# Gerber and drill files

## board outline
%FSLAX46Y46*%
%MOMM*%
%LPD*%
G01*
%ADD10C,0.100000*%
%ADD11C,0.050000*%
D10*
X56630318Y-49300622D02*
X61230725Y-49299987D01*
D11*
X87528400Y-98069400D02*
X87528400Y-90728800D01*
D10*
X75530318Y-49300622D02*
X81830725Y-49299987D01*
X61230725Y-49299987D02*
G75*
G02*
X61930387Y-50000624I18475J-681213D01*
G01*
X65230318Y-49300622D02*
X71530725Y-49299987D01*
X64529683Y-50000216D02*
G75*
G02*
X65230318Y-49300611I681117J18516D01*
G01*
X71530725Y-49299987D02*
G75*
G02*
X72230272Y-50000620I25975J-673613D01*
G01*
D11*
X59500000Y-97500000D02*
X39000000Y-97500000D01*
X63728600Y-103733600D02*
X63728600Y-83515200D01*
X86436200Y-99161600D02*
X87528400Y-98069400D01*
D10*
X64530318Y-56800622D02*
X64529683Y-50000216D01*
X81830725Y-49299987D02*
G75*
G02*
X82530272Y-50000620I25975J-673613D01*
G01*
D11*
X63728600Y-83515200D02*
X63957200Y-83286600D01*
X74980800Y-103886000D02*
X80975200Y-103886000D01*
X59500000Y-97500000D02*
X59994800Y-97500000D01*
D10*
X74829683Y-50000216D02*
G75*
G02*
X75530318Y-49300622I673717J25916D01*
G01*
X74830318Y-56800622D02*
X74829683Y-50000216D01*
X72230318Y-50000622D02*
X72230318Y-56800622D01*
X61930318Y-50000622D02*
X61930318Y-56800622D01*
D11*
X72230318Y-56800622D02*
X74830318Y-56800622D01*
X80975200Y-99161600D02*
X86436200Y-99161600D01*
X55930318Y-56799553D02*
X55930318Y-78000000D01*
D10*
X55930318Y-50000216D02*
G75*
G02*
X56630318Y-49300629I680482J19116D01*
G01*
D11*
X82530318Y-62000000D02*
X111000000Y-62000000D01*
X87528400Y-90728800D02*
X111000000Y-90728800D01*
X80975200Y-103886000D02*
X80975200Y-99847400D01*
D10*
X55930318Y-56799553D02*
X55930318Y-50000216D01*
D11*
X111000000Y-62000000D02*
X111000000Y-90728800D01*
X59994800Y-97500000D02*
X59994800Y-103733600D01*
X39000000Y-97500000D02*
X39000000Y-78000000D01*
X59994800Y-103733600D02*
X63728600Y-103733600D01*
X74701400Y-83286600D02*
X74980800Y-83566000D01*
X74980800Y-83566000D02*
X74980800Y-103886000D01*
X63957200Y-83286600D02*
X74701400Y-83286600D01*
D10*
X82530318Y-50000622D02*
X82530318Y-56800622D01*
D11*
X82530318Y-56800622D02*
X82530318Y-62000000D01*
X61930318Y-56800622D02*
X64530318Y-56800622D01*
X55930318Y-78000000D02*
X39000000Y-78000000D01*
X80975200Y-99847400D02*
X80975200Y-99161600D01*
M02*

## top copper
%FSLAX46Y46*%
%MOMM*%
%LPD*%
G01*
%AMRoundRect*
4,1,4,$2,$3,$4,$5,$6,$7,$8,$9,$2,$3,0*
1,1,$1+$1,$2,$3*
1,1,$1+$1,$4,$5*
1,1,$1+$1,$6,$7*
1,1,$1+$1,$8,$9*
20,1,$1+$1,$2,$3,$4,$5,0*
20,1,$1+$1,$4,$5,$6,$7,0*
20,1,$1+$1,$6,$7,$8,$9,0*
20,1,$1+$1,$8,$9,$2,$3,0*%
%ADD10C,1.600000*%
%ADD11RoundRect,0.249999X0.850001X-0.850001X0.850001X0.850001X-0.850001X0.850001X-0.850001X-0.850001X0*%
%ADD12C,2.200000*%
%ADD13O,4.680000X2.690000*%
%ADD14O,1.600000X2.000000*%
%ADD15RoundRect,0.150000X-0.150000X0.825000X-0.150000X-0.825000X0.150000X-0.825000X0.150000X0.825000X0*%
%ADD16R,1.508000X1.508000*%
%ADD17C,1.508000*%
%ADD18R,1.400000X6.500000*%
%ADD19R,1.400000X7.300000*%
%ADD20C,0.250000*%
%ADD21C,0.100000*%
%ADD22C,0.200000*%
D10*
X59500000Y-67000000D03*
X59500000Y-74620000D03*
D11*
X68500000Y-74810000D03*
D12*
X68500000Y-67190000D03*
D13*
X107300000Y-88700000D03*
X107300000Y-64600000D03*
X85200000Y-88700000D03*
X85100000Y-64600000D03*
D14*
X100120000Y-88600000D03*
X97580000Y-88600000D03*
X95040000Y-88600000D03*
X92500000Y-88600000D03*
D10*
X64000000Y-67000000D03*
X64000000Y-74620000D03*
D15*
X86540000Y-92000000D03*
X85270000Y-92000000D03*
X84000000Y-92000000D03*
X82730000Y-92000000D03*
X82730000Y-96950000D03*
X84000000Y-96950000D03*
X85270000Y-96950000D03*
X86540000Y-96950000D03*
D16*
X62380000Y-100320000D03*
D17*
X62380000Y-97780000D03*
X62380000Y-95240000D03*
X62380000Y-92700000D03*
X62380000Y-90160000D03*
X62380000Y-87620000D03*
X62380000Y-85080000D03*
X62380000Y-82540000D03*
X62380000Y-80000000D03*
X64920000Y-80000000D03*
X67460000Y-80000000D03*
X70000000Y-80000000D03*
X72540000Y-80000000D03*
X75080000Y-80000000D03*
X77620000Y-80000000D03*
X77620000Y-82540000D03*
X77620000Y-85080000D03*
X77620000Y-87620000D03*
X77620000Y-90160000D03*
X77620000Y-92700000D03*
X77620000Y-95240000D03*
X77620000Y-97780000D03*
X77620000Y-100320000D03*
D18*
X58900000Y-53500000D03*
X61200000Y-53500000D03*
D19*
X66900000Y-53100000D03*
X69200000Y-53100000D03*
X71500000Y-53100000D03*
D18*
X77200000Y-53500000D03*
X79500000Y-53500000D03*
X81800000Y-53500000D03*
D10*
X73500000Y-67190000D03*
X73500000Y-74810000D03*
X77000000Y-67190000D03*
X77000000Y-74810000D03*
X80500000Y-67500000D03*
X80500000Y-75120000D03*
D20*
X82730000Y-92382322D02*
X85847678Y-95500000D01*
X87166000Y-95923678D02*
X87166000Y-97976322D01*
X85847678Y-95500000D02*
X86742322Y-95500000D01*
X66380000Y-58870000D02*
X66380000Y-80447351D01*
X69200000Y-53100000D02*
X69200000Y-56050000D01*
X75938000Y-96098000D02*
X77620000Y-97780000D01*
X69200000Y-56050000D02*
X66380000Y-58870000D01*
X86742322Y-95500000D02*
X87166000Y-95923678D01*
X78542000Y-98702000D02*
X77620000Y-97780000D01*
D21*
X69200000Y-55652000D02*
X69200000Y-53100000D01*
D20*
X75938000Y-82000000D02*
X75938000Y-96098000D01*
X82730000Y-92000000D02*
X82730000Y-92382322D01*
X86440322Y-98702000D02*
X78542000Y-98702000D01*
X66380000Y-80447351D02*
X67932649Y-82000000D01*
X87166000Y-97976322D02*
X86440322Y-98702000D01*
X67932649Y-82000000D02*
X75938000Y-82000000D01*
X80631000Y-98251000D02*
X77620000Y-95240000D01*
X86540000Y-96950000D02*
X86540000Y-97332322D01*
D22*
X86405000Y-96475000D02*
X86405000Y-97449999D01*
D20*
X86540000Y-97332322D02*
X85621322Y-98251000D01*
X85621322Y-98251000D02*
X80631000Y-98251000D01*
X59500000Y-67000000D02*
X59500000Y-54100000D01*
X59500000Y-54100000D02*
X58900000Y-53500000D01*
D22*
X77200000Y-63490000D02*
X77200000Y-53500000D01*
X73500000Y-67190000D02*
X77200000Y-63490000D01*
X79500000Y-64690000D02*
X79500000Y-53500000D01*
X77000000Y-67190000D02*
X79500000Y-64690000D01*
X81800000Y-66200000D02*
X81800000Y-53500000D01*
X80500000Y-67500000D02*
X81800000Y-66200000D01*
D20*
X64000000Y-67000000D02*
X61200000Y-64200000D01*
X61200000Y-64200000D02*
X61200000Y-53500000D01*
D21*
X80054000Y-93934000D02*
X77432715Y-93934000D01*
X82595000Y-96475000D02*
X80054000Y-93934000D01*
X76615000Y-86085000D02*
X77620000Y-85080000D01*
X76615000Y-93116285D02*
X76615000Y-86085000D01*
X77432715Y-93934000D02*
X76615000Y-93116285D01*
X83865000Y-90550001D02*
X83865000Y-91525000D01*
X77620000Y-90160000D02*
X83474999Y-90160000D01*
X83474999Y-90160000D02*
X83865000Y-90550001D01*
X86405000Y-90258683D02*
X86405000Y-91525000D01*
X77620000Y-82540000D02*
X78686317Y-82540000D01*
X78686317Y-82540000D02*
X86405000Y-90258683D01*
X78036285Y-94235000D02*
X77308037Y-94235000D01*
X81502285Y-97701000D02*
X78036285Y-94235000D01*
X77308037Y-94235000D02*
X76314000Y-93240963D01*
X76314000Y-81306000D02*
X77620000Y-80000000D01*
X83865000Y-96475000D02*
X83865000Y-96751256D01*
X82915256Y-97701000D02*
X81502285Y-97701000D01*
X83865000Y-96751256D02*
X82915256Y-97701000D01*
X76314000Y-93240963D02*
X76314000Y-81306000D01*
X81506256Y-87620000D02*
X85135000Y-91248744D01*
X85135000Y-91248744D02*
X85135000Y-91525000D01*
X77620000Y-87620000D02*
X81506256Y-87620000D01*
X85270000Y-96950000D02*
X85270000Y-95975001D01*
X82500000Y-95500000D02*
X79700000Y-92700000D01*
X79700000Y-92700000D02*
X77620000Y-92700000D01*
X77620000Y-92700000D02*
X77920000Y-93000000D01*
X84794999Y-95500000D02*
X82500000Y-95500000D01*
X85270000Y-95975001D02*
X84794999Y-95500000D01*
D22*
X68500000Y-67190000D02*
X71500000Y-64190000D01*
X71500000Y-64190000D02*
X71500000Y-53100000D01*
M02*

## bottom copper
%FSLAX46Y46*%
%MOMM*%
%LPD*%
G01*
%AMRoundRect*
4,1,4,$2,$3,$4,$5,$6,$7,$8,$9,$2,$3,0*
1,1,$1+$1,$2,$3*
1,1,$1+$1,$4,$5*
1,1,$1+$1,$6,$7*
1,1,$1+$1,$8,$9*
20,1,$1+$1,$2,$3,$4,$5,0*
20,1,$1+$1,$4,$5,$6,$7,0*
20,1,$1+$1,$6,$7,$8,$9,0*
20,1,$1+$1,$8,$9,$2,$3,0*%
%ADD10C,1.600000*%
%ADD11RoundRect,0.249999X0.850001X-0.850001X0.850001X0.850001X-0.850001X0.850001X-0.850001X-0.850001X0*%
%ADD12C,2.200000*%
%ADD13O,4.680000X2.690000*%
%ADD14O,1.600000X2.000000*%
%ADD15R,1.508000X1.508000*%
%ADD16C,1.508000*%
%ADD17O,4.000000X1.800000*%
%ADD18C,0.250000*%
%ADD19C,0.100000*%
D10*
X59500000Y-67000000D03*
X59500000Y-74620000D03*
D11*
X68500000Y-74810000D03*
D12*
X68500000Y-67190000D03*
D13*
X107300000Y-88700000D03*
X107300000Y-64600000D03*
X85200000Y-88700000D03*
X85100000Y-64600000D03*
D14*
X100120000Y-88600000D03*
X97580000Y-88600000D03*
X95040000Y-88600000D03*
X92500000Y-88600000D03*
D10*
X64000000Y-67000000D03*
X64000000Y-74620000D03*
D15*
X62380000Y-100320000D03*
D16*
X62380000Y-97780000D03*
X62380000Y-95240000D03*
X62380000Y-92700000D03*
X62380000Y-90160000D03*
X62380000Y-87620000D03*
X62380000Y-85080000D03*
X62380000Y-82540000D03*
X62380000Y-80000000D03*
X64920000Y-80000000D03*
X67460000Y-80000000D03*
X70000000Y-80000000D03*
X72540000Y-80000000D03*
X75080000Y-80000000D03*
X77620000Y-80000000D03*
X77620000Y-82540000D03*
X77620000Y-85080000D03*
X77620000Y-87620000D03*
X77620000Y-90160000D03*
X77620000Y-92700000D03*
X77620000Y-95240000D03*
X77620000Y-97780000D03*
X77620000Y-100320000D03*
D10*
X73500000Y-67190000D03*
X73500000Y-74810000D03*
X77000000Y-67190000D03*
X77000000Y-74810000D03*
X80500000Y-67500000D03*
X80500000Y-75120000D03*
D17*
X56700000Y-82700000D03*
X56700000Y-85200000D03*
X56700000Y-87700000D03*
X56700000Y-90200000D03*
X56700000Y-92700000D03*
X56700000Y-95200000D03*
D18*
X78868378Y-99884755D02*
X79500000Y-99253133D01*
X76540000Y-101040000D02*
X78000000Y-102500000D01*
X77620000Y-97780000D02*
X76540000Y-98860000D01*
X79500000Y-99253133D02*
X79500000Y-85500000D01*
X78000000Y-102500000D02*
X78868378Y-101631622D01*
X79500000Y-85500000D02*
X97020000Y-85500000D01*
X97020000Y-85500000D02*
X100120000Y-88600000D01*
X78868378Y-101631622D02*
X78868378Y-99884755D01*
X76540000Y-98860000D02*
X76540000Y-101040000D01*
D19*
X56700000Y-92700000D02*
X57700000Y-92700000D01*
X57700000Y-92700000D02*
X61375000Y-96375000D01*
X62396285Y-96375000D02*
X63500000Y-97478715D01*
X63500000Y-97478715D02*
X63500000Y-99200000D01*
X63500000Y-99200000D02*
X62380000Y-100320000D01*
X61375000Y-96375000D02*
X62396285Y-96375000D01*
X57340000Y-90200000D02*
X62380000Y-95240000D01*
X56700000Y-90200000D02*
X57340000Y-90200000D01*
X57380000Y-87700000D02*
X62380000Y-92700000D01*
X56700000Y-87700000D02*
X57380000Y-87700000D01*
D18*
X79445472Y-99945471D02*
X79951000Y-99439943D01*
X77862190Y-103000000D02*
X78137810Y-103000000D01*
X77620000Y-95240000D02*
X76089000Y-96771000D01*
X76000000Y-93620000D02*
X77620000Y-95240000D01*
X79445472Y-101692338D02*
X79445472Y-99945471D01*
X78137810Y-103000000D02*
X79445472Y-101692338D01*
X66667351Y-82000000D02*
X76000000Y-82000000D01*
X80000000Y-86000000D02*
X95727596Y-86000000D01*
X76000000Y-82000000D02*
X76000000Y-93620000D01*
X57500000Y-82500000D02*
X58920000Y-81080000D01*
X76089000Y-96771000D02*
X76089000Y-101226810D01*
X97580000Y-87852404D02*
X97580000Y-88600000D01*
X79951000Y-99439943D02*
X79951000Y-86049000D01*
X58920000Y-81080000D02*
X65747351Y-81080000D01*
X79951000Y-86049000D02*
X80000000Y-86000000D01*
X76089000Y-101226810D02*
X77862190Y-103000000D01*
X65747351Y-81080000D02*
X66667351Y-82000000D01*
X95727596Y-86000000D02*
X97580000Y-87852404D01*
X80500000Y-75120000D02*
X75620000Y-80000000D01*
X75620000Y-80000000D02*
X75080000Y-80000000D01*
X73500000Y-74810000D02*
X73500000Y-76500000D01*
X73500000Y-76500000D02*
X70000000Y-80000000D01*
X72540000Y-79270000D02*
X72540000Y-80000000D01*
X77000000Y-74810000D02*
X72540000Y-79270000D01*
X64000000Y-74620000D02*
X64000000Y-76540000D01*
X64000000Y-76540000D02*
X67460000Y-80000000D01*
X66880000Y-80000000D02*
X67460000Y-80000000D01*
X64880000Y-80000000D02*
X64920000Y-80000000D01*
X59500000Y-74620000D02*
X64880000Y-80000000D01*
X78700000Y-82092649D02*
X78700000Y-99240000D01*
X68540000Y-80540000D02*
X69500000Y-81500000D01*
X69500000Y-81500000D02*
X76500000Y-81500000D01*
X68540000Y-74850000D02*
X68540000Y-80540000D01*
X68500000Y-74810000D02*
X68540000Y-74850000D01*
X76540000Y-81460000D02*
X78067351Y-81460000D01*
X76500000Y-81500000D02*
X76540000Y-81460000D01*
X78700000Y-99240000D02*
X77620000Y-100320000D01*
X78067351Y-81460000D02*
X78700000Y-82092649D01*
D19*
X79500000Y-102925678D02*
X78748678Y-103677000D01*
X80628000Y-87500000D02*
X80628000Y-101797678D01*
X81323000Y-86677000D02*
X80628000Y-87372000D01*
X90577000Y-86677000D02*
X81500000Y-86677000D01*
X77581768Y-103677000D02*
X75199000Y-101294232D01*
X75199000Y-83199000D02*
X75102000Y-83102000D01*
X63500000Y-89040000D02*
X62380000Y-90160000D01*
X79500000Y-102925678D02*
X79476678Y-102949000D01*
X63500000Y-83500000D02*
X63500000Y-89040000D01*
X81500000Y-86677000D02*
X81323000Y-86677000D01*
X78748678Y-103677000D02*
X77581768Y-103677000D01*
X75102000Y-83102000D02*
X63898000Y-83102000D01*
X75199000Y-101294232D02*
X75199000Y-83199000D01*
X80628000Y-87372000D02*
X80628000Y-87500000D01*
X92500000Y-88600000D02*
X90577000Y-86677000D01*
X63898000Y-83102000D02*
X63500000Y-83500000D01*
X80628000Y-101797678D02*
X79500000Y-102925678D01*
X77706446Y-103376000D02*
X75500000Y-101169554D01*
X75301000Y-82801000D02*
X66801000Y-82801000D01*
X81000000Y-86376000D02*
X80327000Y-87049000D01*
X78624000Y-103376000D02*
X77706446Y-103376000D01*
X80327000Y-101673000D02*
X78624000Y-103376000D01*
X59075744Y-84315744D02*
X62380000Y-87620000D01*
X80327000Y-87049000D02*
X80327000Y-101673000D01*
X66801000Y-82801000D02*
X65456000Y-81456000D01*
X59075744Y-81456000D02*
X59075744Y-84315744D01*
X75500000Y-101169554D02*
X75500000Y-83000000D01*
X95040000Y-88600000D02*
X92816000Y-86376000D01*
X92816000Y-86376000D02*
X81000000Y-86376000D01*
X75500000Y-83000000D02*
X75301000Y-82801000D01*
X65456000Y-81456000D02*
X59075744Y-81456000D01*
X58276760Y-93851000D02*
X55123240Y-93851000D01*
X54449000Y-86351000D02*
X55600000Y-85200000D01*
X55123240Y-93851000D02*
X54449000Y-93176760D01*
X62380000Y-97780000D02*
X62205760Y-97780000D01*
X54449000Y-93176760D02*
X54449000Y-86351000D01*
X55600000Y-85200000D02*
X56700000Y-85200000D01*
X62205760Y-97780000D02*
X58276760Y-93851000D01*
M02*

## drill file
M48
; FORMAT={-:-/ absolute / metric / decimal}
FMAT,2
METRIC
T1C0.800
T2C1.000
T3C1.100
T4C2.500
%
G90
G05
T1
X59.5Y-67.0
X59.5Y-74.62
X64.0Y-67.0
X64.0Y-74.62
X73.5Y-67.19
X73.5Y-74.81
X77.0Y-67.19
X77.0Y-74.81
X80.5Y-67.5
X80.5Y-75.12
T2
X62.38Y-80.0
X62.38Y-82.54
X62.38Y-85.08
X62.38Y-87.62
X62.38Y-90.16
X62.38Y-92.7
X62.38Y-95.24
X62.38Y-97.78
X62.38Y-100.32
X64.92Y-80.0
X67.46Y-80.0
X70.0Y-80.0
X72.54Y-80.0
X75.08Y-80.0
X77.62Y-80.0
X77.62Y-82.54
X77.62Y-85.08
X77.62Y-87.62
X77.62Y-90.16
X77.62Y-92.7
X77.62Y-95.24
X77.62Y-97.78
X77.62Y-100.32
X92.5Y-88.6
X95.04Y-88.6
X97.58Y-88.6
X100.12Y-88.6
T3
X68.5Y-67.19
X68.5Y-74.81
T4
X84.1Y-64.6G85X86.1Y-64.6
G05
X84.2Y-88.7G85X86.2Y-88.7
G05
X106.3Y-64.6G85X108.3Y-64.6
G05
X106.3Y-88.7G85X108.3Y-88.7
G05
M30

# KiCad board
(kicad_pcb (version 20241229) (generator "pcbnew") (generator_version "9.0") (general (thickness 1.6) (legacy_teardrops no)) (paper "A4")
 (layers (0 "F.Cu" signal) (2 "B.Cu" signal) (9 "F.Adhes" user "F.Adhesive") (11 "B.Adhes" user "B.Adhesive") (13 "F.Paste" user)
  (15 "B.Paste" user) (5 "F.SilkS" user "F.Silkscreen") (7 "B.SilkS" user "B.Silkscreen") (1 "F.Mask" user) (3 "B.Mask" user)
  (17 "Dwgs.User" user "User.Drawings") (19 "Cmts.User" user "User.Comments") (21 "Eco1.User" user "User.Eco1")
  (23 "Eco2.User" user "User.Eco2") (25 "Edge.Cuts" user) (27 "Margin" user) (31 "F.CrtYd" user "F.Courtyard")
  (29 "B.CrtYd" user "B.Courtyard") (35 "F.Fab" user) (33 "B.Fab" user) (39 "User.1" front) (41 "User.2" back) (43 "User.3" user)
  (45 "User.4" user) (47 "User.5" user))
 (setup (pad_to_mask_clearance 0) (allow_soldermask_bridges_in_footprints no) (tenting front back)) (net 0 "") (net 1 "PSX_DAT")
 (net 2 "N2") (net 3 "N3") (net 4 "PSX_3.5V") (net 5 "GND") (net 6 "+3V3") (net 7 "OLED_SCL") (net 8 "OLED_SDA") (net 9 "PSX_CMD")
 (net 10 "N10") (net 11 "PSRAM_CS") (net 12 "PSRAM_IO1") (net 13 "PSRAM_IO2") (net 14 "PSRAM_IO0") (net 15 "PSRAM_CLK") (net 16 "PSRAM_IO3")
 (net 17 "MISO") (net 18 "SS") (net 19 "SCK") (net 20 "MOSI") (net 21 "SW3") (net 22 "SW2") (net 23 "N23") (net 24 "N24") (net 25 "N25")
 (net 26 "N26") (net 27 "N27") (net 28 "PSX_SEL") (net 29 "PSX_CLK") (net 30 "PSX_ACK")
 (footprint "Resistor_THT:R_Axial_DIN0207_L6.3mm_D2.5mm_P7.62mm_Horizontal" (layer "F.Cu") (at 59.5 67 -90)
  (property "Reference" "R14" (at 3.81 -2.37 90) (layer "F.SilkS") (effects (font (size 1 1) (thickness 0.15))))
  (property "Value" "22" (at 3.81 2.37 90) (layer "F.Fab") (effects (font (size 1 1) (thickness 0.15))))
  (pad "1" thru_hole circle (at 0 0 270) (size 1.6 1.6) (drill 0.8) (layers "*.Cu" "*.Mask") (remove_unused_layers no) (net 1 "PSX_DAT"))
  (pad "2" thru_hole circle (at 7.62 0 270) (size 1.6 1.6) (drill 0.8) (layers "*.Cu" "*.Mask") (remove_unused_layers no) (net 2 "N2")))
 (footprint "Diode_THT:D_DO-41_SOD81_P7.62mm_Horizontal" (layer "F.Cu") (at 68.5 74.81 90)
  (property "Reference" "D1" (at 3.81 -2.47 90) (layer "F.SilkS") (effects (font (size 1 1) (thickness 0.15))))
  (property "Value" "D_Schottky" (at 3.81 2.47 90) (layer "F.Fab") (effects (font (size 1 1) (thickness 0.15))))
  (pad "1" thru_hole roundrect (at 0 0 90) (size 2.2 2.2) (drill 1.1) (layers "*.Cu" "*.Mask") (remove_unused_layers no)
   (roundrect_rratio 0.113636) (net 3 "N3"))
  (pad "2" thru_hole circle (at 7.62 0 90) (size 2.2 2.2) (drill 1.1) (layers "*.Cu" "*.Mask") (remove_unused_layers no) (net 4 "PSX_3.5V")))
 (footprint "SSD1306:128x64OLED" (layer "F.Cu") (at 96.5 78 180)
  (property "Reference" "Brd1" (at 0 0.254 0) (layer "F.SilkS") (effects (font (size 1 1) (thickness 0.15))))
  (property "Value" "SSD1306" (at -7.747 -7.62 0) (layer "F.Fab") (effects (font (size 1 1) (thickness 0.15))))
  (pad "" thru_hole oval (at -10.8 -10.7) (size 4.68 2.69) (drill oval 4.5 2.5) (layers "*.Cu" "*.Mask") (remove_unused_layers no))
  (pad "" thru_hole oval (at -10.8 13.4) (size 4.68 2.69) (drill oval 4.5 2.5) (layers "*.Cu" "*.Mask") (remove_unused_layers no))
  (pad "" thru_hole oval (at 11.3 -10.7) (size 4.68 2.69) (drill oval 4.5 2.5) (layers "*.Cu" "*.Mask") (remove_unused_layers no))
  (pad "" thru_hole oval (at 11.4 13.4) (size 4.68 2.69) (drill oval 4.5 2.5) (layers "*.Cu" "*.Mask") (remove_unused_layers no))
  (pad "1" thru_hole oval (at -3.62 -10.6 270) (size 2 1.6) (drill 1) (layers "*.Cu" "*.Mask") (remove_unused_layers no) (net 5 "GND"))
  (pad "2" thru_hole oval (at -1.08 -10.6 270) (size 2 1.6) (drill 1) (layers "*.Cu" "*.Mask") (remove_unused_layers no) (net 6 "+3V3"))
  (pad "3" thru_hole oval (at 1.46 -10.6 270) (size 2 1.6) (drill 1) (layers "*.Cu" "*.Mask") (remove_unused_layers no) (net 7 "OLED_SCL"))
  (pad "4" thru_hole oval (at 4 -10.6 270) (size 2 1.6) (drill 1) (layers "*.Cu" "*.Mask") (remove_unused_layers no) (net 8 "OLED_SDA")))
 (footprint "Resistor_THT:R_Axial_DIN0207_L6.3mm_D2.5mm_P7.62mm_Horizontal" (layer "F.Cu") (at 64 67 -90)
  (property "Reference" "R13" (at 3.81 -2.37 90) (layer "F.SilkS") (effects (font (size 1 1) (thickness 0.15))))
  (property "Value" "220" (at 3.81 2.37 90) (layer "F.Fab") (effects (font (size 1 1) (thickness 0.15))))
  (pad "1" thru_hole circle (at 0 0 270) (size 1.6 1.6) (drill 0.8) (layers "*.Cu" "*.Mask") (remove_unused_layers no) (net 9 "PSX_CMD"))
  (pad "2" thru_hole circle (at 7.62 0 270) (size 1.6 1.6) (drill 0.8) (layers "*.Cu" "*.Mask") (remove_unused_layers no) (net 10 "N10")))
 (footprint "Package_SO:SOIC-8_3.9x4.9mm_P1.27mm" (layer "F.Cu") (at 84.635 94.475 -90)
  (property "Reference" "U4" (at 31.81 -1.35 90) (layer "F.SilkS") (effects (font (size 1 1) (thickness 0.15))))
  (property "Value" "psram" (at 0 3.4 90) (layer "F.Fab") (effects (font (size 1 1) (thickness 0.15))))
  (pad "1" smd roundrect (at -2.475 -1.905 270) (size 1.95 0.6) (layers "F.Cu" "F.Mask" "F.Paste") (roundrect_rratio 0.25)
   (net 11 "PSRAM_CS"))
  (pad "2" smd roundrect (at -2.475 -0.635 270) (size 1.95 0.6) (layers "F.Cu" "F.Mask" "F.Paste") (roundrect_rratio 0.25)
   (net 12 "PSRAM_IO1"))
  (pad "3" smd roundrect (at -2.475 0.635 270) (size 1.95 0.6) (layers "F.Cu" "F.Mask" "F.Paste") (roundrect_rratio 0.25)
   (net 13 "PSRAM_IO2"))
  (pad "4" smd roundrect (at -2.475 1.905 270) (size 1.95 0.6) (layers "F.Cu" "F.Mask" "F.Paste") (roundrect_rratio 0.25) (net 5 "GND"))
  (pad "5" smd roundrect (at 2.475 1.905 270) (size 1.95 0.6) (layers "F.Cu" "F.Mask" "F.Paste") (roundrect_rratio 0.25)
   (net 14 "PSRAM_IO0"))
  (pad "6" smd roundrect (at 2.475 0.635 270) (size 1.95 0.6) (layers "F.Cu" "F.Mask" "F.Paste") (roundrect_rratio 0.25)
   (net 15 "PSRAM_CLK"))
  (pad "7" smd roundrect (at 2.475 -0.635 270) (size 1.95 0.6) (layers "F.Cu" "F.Mask" "F.Paste") (roundrect_rratio 0.25)
   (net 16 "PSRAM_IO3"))
  (pad "8" smd roundrect (at 2.475 -1.905 270) (size 1.95 0.6) (layers "F.Cu" "F.Mask" "F.Paste") (roundrect_rratio 0.25) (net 6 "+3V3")))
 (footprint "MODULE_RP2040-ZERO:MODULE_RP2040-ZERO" (layer "F.Cu") (at 70 90.16 180)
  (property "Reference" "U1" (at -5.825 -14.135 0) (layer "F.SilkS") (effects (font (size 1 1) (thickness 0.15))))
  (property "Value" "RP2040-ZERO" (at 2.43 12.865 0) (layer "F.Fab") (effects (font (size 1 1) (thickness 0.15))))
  (pad "1" thru_hole rect (at 7.62 -10.16 180) (size 1.508 1.508) (drill 1) (layers "*.Cu" "*.Mask") (remove_unused_layers no)
   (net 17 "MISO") (solder_mask_margin 0.102))
  (pad "2" thru_hole circle (at 7.62 -7.62 180) (size 1.508 1.508) (drill 1) (layers "*.Cu" "*.Mask") (remove_unused_layers no)
   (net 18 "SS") (solder_mask_margin 0.102))
  (pad "3" thru_hole circle (at 7.62 -5.08 180) (size 1.508 1.508) (drill 1) (layers "*.Cu" "*.Mask") (remove_unused_layers no)
   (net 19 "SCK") (solder_mask_margin 0.102))
  (pad "4" thru_hole circle (at 7.62 -2.54 180) (size 1.508 1.508) (drill 1) (layers "*.Cu" "*.Mask") (remove_unused_layers no)
   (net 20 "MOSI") (solder_mask_margin 0.102))
  (pad "5" thru_hole circle (at 7.62 0 180) (size 1.508 1.508) (drill 1) (layers "*.Cu" "*.Mask") (remove_unused_layers no)
   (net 8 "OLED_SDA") (solder_mask_margin 0.102))
  (pad "6" thru_hole circle (at 7.62 2.54 180) (size 1.508 1.508) (drill 1) (layers "*.Cu" "*.Mask") (remove_unused_layers no)
   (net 7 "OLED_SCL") (solder_mask_margin 0.102))
  (pad "7" thru_hole circle (at 7.62 5.08 180) (size 1.508 1.508) (drill 1) (layers "*.Cu" "*.Mask") (remove_unused_layers no)
   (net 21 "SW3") (solder_mask_margin 0.102))
  (pad "8" thru_hole circle (at 7.62 7.62 180) (size 1.508 1.508) (drill 1) (layers "*.Cu" "*.Mask") (remove_unused_layers no)
   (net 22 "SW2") (solder_mask_margin 0.102))
  (pad "9" thru_hole circle (at 7.62 10.16 180) (size 1.508 1.508) (drill 1) (layers "*.Cu" "*.Mask") (remove_unused_layers no)
   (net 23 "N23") (solder_mask_margin 0.102))
  (pad "10" thru_hole circle (at 5.08 10.16 180) (size 1.508 1.508) (drill 1) (layers "*.Cu" "*.Mask") (remove_unused_layers no)
   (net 2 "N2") (solder_mask_margin 0.102))
  (pad "11" thru_hole circle (at 2.54 10.16 180) (size 1.508 1.508) (drill 1) (layers "*.Cu" "*.Mask") (remove_unused_layers no)
   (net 10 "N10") (solder_mask_margin 0.102))
  (pad "12" thru_hole circle (at 0 10.16 180) (size 1.508 1.508) (drill 1) (layers "*.Cu" "*.Mask") (remove_unused_layers no) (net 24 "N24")
   (solder_mask_margin 0.102))
  (pad "13" thru_hole circle (at -2.54 10.16 180) (size 1.508 1.508) (drill 1) (layers "*.Cu" "*.Mask") (remove_unused_layers no)
   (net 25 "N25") (solder_mask_margin 0.102))
  (pad "14" thru_hole circle (at -5.08 10.16 180) (size 1.508 1.508) (drill 1) (layers "*.Cu" "*.Mask") (remove_unused_layers no)
   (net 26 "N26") (solder_mask_margin 0.102))
  (pad "15" thru_hole circle (at -7.62 10.16 180) (size 1.508 1.508) (drill 1) (layers "*.Cu" "*.Mask") (remove_unused_layers no)
   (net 15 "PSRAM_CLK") (solder_mask_margin 0.102))
  (pad "16" thru_hole circle (at -7.62 7.62 180) (size 1.508 1.508) (drill 1) (layers "*.Cu" "*.Mask") (remove_unused_layers no)
   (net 11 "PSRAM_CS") (solder_mask_margin 0.102))
  (pad "17" thru_hole circle (at -7.62 5.08 180) (size 1.508 1.508) (drill 1) (layers "*.Cu" "*.Mask") (remove_unused_layers no)
   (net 14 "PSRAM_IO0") (solder_mask_margin 0.102))
  (pad "18" thru_hole circle (at -7.62 2.54 180) (size 1.508 1.508) (drill 1) (layers "*.Cu" "*.Mask") (remove_unused_layers no)
   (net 12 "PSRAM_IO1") (solder_mask_margin 0.102))
  (pad "19" thru_hole circle (at -7.62 0 180) (size 1.508 1.508) (drill 1) (layers "*.Cu" "*.Mask") (remove_unused_layers no)
   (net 13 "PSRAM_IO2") (solder_mask_margin 0.102))
  (pad "20" thru_hole circle (at -7.62 -2.54 180) (size 1.508 1.508) (drill 1) (layers "*.Cu" "*.Mask") (remove_unused_layers no)
   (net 16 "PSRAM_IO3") (solder_mask_margin 0.102))
  (pad "21" thru_hole circle (at -7.62 -5.08 180) (size 1.508 1.508) (drill 1) (layers "*.Cu" "*.Mask") (remove_unused_layers no)
   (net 6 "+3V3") (solder_mask_margin 0.102))
  (pad "22" thru_hole circle (at -7.62 -7.62 180) (size 1.508 1.508) (drill 1) (layers "*.Cu" "*.Mask") (remove_unused_layers no)
   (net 5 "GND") (solder_mask_margin 0.102))
  (pad "23" thru_hole circle (at -7.62 -10.16 180) (size 1.508 1.508) (drill 1) (layers "*.Cu" "*.Mask") (remove_unused_layers no)
   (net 3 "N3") (solder_mask_margin 0.102)))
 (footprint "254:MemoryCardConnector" (layer "F.Cu") (at 69.2 53.1)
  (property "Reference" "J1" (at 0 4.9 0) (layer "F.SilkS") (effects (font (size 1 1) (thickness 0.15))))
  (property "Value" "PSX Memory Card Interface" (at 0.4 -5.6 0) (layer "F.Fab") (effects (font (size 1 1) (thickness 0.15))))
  (pad "1" smd rect (at -10.3 0.4) (size 1.4 6.5) (layers "F.Cu" "F.Mask" "F.Paste") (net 1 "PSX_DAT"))
  (pad "2" smd rect (at -8 0.4) (size 1.4 6.5) (layers "F.Cu" "F.Mask" "F.Paste") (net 9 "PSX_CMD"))
  (pad "3" smd rect (at -2.3 0) (size 1.4 7.3) (layers "F.Cu" "F.Mask" "F.Paste") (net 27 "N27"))
  (pad "4" smd rect (at 0 0) (size 1.4 7.3) (layers "F.Cu" "F.Mask" "F.Paste") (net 5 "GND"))
  (pad "5" smd rect (at 2.3 0) (size 1.4 7.3) (layers "F.Cu" "F.Mask" "F.Paste") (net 4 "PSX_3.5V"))
  (pad "6" smd rect (at 8 0.4) (size 1.4 6.5) (layers "F.Cu" "F.Mask" "F.Paste") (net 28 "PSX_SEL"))
  (pad "7" smd rect (at 10.3 0.4) (size 1.4 6.5) (layers "F.Cu" "F.Mask" "F.Paste") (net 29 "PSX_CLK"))
  (pad "8" smd rect (at 12.6 0.4) (size 1.4 6.5) (layers "F.Cu" "F.Mask" "F.Paste") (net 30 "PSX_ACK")))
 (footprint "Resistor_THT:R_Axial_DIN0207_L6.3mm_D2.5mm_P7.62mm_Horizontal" (layer "F.Cu") (at 73.5 67.19 -90)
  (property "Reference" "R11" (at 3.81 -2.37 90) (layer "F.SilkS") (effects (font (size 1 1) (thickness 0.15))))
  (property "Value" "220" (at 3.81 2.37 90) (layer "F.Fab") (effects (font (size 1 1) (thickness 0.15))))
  (pad "1" thru_hole circle (at 0 0 270) (size 1.6 1.6) (drill 0.8) (layers "*.Cu" "*.Mask") (remove_unused_layers no) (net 28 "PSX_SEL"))
  (pad "2" thru_hole circle (at 7.62 0 270) (size 1.6 1.6) (drill 0.8) (layers "*.Cu" "*.Mask") (remove_unused_layers no) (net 24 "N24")))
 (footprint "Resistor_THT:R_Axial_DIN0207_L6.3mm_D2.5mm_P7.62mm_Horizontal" (layer "F.Cu") (at 77 67.19 -90)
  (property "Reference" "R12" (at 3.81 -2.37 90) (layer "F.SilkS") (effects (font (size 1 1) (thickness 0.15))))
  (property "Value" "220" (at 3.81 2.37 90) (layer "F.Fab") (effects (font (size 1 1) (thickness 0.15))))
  (pad "1" thru_hole circle (at 0 0 270) (size 1.6 1.6) (drill 0.8) (layers "*.Cu" "*.Mask") (remove_unused_layers no) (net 29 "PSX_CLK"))
  (pad "2" thru_hole circle (at 7.62 0 270) (size 1.6 1.6) (drill 0.8) (layers "*.Cu" "*.Mask") (remove_unused_layers no) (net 25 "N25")))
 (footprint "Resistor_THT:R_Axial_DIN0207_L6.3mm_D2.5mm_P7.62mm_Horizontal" (layer "F.Cu") (at 80.5 67.5 -90)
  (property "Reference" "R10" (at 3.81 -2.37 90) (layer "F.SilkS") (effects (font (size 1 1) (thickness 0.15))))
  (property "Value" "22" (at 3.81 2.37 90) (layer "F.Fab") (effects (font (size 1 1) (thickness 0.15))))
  (pad "1" thru_hole circle (at 0 0 270) (size 1.6 1.6) (drill 0.8) (layers "*.Cu" "*.Mask") (remove_unused_layers no) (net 30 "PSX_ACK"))
  (pad "2" thru_hole circle (at 7.62 0 270) (size 1.6 1.6) (drill 0.8) (layers "*.Cu" "*.Mask") (remove_unused_layers no) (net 26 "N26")))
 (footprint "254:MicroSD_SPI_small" (layer "B.Cu") (at 55.5 89)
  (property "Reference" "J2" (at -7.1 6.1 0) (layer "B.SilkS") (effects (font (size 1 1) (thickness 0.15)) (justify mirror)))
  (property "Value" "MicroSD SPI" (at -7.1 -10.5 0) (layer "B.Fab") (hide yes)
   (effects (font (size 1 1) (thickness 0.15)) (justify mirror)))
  (pad "1" smd oval (at 1.2 -6.3) (size 4 1.8) (layers "B.Cu" "B.Mask" "B.Paste") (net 6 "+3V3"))
  (pad "2" smd oval (at 1.2 -3.8) (size 4 1.8) (layers "B.Cu" "B.Mask" "B.Paste") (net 18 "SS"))
  (pad "3" smd oval (at 1.2 -1.3) (size 4 1.8) (layers "B.Cu" "B.Mask" "B.Paste") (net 20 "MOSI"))
  (pad "4" smd oval (at 1.2 1.2) (size 4 1.8) (layers "B.Cu" "B.Mask" "B.Paste") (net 19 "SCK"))
  (pad "5" smd oval (at 1.2 3.7) (size 4 1.8) (layers "B.Cu" "B.Mask" "B.Paste") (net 17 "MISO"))
  (pad "6" smd oval (at 1.2 6.2) (size 4 1.8) (layers "B.Cu" "B.Mask" "B.Paste") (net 5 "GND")))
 (gr_line (start 56.630318 49.300622) (end 61.230725 49.299987) (stroke (width 0.1) (type solid)) (layer "Edge.Cuts"))
 (gr_line (start 87.5284 98.0694) (end 87.5284 90.7288) (stroke (width 0.05) (type default)) (layer "Edge.Cuts"))
 (gr_line (start 75.530318 49.300622) (end 81.830725 49.299987) (stroke (width 0.1) (type solid)) (layer "Edge.Cuts"))
 (gr_arc (start 61.230725 49.299987) (mid 61.731367 49.499673) (end 61.930318 50.000622) (stroke (width 0.1) (type solid))
  (layer "Edge.Cuts"))
 (gr_line (start 65.230318 49.300622) (end 71.530725 49.299987) (stroke (width 0.1) (type solid)) (layer "Edge.Cuts"))
 (gr_arc (start 64.529683 50.000216) (mid 64.729354 49.499545) (end 65.230318 49.300622) (stroke (width 0.1) (type solid))
  (layer "Edge.Cuts"))
 (gr_arc (start 71.530725 49.299987) (mid 72.033777 49.497295) (end 72.230318 50.000622) (stroke (width 0.1) (type solid))
  (layer "Edge.Cuts"))
 (gr_line (start 59.5 97.5) (end 39 97.5) (stroke (width 0.05) (type default)) (layer "Edge.Cuts"))
 (gr_line (start 63.7286 103.7336) (end 63.7286 83.5152) (stroke (width 0.05) (type default)) (layer "Edge.Cuts"))
 (gr_line (start 86.4362 99.1616) (end 87.5284 98.0694) (stroke (width 0.05) (type default)) (layer "Edge.Cuts"))
 (gr_line (start 64.530318 56.800622) (end 64.529683 50.000216) (stroke (width 0.1) (type solid)) (layer "Edge.Cuts"))
 (gr_arc (start 81.830725 49.299987) (mid 82.333777 49.497295) (end 82.530318 50.000622) (stroke (width 0.1) (type solid))
  (layer "Edge.Cuts"))
 (gr_line (start 63.7286 83.5152) (end 63.9572 83.2866) (stroke (width 0.05) (type default)) (layer "Edge.Cuts"))
 (gr_line (start 74.9808 103.886) (end 80.9752 103.886) (stroke (width 0.05) (type default)) (layer "Edge.Cuts"))
 (gr_line (start 59.5 97.5) (end 59.9948 97.5) (stroke (width 0.05) (type default)) (layer "Edge.Cuts"))
 (gr_arc (start 74.829683 50.000216) (mid 75.027012 49.497203) (end 75.530318 49.300622) (stroke (width 0.1) (type solid))
  (layer "Edge.Cuts"))
 (gr_line (start 74.830318 56.800622) (end 74.829683 50.000216) (stroke (width 0.1) (type solid)) (layer "Edge.Cuts"))
 (gr_line (start 72.230318 50.000622) (end 72.230318 56.800622) (stroke (width 0.1) (type solid)) (layer "Edge.Cuts"))
 (gr_line (start 61.930318 50.000622) (end 61.930318 56.800622) (stroke (width 0.1) (type solid)) (layer "Edge.Cuts"))
 (gr_line (start 72.230318 56.800622) (end 74.830318 56.800622) (stroke (width 0.05) (type default)) (layer "Edge.Cuts"))
 (gr_line (start 80.9752 99.1616) (end 86.4362 99.1616) (stroke (width 0.05) (type default)) (layer "Edge.Cuts"))
 (gr_line (start 55.930318 56.799553) (end 55.930318 78) (stroke (width 0.05) (type default)) (layer "Edge.Cuts"))
 (gr_arc (start 55.930318 50.000216) (mid 56.129579 49.499595) (end 56.630318 49.300622) (stroke (width 0.1) (type solid))
  (layer "Edge.Cuts"))
 (gr_line (start 82.530318 62) (end 111 62) (stroke (width 0.05) (type default)) (layer "Edge.Cuts"))
 (gr_line (start 87.5284 90.7288) (end 111 90.7288) (stroke (width 0.05) (type default)) (layer "Edge.Cuts"))
 (gr_line (start 80.9752 103.886) (end 80.9752 99.8474) (stroke (width 0.05) (type default)) (layer "Edge.Cuts"))
 (gr_line (start 55.930318 56.799553) (end 55.930318 50.000216) (stroke (width 0.1) (type solid)) (layer "Edge.Cuts"))
 (gr_line (start 111 62) (end 111 90.7288) (stroke (width 0.05) (type default)) (layer "Edge.Cuts"))
 (gr_line (start 59.9948 97.5) (end 59.9948 103.7336) (stroke (width 0.05) (type default)) (layer "Edge.Cuts"))
 (gr_line (start 39 97.5) (end 39 78) (stroke (width 0.05) (type default)) (layer "Edge.Cuts"))
 (gr_line (start 59.9948 103.7336) (end 63.7286 103.7336) (stroke (width 0.05) (type default)) (layer "Edge.Cuts"))
 (gr_line (start 74.7014 83.2866) (end 74.9808 83.566) (stroke (width 0.05) (type default)) (layer "Edge.Cuts"))
 (gr_line (start 74.9808 83.566) (end 74.9808 103.886) (stroke (width 0.05) (type default)) (layer "Edge.Cuts"))
 (gr_line (start 63.9572 83.2866) (end 74.7014 83.2866) (stroke (width 0.05) (type default)) (layer "Edge.Cuts"))
 (gr_line (start 82.530318 50.000622) (end 82.530318 56.800622) (stroke (width 0.1) (type solid)) (layer "Edge.Cuts"))
 (gr_line (start 82.530318 56.800622) (end 82.530318 62) (stroke (width 0.05) (type default)) (layer "Edge.Cuts"))
 (gr_line (start 61.930318 56.800622) (end 64.530318 56.800622) (stroke (width 0.05) (type default)) (layer "Edge.Cuts"))
 (gr_line (start 55.930318 78) (end 39 78) (stroke (width 0.05) (type default)) (layer "Edge.Cuts"))
 (gr_line (start 80.9752 99.8474) (end 80.9752 99.1616) (stroke (width 0.05) (type default)) (layer "Edge.Cuts"))
 (segment (start 82.73 92.382322) (end 85.847678 95.5) (width 0.25) (layer "F.Cu") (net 5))
 (segment (start 87.166 95.923678) (end 87.166 97.976322) (width 0.25) (layer "F.Cu") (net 5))
 (segment (start 85.847678 95.5) (end 86.742322 95.5) (width 0.25) (layer "F.Cu") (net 5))
 (segment (start 66.38 58.87) (end 66.38 80.447351) (width 0.25) (layer "F.Cu") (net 5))
 (segment (start 69.2 53.1) (end 69.2 56.05) (width 0.25) (layer "F.Cu") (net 5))
 (segment (start 75.938 96.098) (end 77.62 97.78) (width 0.25) (layer "F.Cu") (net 5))
 (segment (start 69.2 56.05) (end 66.38 58.87) (width 0.25) (layer "F.Cu") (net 5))
 (segment (start 86.742322 95.5) (end 87.166 95.923678) (width 0.25) (layer "F.Cu") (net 5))
 (segment (start 78.542 98.702) (end 77.62 97.78) (width 0.25) (layer "F.Cu") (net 5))
 (segment (start 69.2 55.652) (end 69.2 53.1) (width 0.1) (layer "F.Cu") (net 5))
 (segment (start 75.938 82) (end 75.938 96.098) (width 0.25) (layer "F.Cu") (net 5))
 (segment (start 82.73 92) (end 82.73 92.382322) (width 0.25) (layer "F.Cu") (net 5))
 (segment (start 86.440322 98.702) (end 78.542 98.702) (width 0.25) (layer "F.Cu") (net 5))
 (segment (start 66.38 80.447351) (end 67.932649 82) (width 0.25) (layer "F.Cu") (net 5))
 (segment (start 87.166 97.976322) (end 86.440322 98.702) (width 0.25) (layer "F.Cu") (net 5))
 (segment (start 67.932649 82) (end 75.938 82) (width 0.25) (layer "F.Cu") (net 5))
 (segment (start 78.868378 99.884755) (end 79.5 99.253133) (width 0.25) (layer "B.Cu") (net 5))
 (segment (start 76.54 101.04) (end 78 102.5) (width 0.25) (layer "B.Cu") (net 5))
 (segment (start 77.62 97.78) (end 76.54 98.86) (width 0.25) (layer "B.Cu") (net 5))
 (segment (start 79.5 99.253133) (end 79.5 85.5) (width 0.25) (layer "B.Cu") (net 5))
 (segment (start 78 102.5) (end 78.868378 101.631622) (width 0.25) (layer "B.Cu") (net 5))
 (segment (start 79.5 85.5) (end 97.02 85.5) (width 0.25) (layer "B.Cu") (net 5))
 (segment (start 97.02 85.5) (end 100.12 88.6) (width 0.25) (layer "B.Cu") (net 5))
 (segment (start 78.868378 101.631622) (end 78.868378 99.884755) (width 0.25) (layer "B.Cu") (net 5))
 (segment (start 76.54 98.86) (end 76.54 101.04) (width 0.25) (layer "B.Cu") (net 5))
 (segment (start 56.7 92.7) (end 57.7 92.7) (width 0.1) (layer "B.Cu") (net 17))
 (segment (start 57.7 92.7) (end 61.375 96.375) (width 0.1) (layer "B.Cu") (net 17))
 (segment (start 62.396285 96.375) (end 63.5 97.478715) (width 0.1) (layer "B.Cu") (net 17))
 (segment (start 63.5 97.478715) (end 63.5 99.2) (width 0.1) (layer "B.Cu") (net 17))
 (segment (start 63.5 99.2) (end 62.38 100.32) (width 0.1) (layer "B.Cu") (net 17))
 (segment (start 61.375 96.375) (end 62.396285 96.375) (width 0.1) (layer "B.Cu") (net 17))
 (segment (start 57.34 90.2) (end 62.38 95.24) (width 0.1) (layer "B.Cu") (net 19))
 (segment (start 56.7 90.2) (end 57.34 90.2) (width 0.1) (layer "B.Cu") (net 19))
 (segment (start 57.38 87.7) (end 62.38 92.7) (width 0.1) (layer "B.Cu") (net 20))
 (segment (start 56.7 87.7) (end 57.38 87.7) (width 0.1) (layer "B.Cu") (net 20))
 (segment (start 80.631 98.251) (end 77.62 95.24) (width 0.25) (layer "F.Cu") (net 6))
 (segment (start 86.54 96.95) (end 86.54 97.332322) (width 0.25) (layer "F.Cu") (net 6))
 (segment (start 86.405 96.475) (end 86.405 97.449999) (width 0.2) (layer "F.Cu") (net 6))
 (segment (start 86.54 97.332322) (end 85.621322 98.251) (width 0.25) (layer "F.Cu") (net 6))
 (segment (start 85.621322 98.251) (end 80.631 98.251) (width 0.25) (layer "F.Cu") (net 6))
 (segment (start 79.445472 99.945471) (end 79.951 99.439943) (width 0.25) (layer "B.Cu") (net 6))
 (segment (start 77.86219 103) (end 78.13781 103) (width 0.25) (layer "B.Cu") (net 6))
 (segment (start 77.62 95.24) (end 76.089 96.771) (width 0.25) (layer "B.Cu") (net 6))
 (segment (start 76 93.62) (end 77.62 95.24) (width 0.25) (layer "B.Cu") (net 6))
 (segment (start 79.445472 101.692338) (end 79.445472 99.945471) (width 0.25) (layer "B.Cu") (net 6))
 (segment (start 78.13781 103) (end 79.445472 101.692338) (width 0.25) (layer "B.Cu") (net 6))
 (segment (start 66.667351 82) (end 76 82) (width 0.25) (layer "B.Cu") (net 6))
 (segment (start 80 86) (end 95.727596 86) (width 0.25) (layer "B.Cu") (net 6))
 (segment (start 76 82) (end 76 93.62) (width 0.25) (layer "B.Cu") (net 6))
 (segment (start 57.5 82.5) (end 58.92 81.08) (width 0.25) (layer "B.Cu") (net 6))
 (segment (start 76.089 96.771) (end 76.089 101.22681) (width 0.25) (layer "B.Cu") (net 6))
 (segment (start 97.58 87.852404) (end 97.58 88.6) (width 0.25) (layer "B.Cu") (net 6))
 (segment (start 79.951 99.439943) (end 79.951 86.049) (width 0.25) (layer "B.Cu") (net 6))
 (segment (start 58.92 81.08) (end 65.747351 81.08) (width 0.25) (layer "B.Cu") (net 6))
 (segment (start 79.951 86.049) (end 80 86) (width 0.25) (layer "B.Cu") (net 6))
 (segment (start 76.089 101.22681) (end 77.86219 103) (width 0.25) (layer "B.Cu") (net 6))
 (segment (start 65.747351 81.08) (end 66.667351 82) (width 0.25) (layer "B.Cu") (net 6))
 (segment (start 95.727596 86) (end 97.58 87.852404) (width 0.25) (layer "B.Cu") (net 6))
 (segment (start 59.5 67) (end 59.5 54.1) (width 0.25) (layer "F.Cu") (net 1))
 (segment (start 59.5 54.1) (end 58.9 53.5) (width 0.25) (layer "F.Cu") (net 1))
 (segment (start 77.2 63.49) (end 77.2 53.5) (width 0.2) (layer "F.Cu") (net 28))
 (segment (start 73.5 67.19) (end 77.2 63.49) (width 0.2) (layer "F.Cu") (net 28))
 (segment (start 79.5 64.69) (end 79.5 53.5) (width 0.2) (layer "F.Cu") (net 29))
 (segment (start 77 67.19) (end 79.5 64.69) (width 0.2) (layer "F.Cu") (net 29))
 (segment (start 81.8 66.2) (end 81.8 53.5) (width 0.2) (layer "F.Cu") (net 30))
 (segment (start 80.5 67.5) (end 81.8 66.2) (width 0.2) (layer "F.Cu") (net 30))
 (segment (start 64 67) (end 61.2 64.2) (width 0.25) (layer "F.Cu") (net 9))
 (segment (start 61.2 64.2) (end 61.2 53.5) (width 0.25) (layer "F.Cu") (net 9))
 (segment (start 80.5 75.12) (end 75.62 80) (width 0.25) (layer "B.Cu") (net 26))
 (segment (start 75.62 80) (end 75.08 80) (width 0.25) (layer "B.Cu") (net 26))
 (segment (start 73.5 74.81) (end 73.5 76.5) (width 0.25) (layer "B.Cu") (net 24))
 (segment (start 73.5 76.5) (end 70 80) (width 0.25) (layer "B.Cu") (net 24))
 (segment (start 72.54 79.27) (end 72.54 80) (width 0.25) (layer "B.Cu") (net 25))
 (segment (start 77 74.81) (end 72.54 79.27) (width 0.25) (layer "B.Cu") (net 25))
 (segment (start 64 74.62) (end 64 76.54) (width 0.25) (layer "B.Cu") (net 10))
 (segment (start 64 76.54) (end 67.46 80) (width 0.25) (layer "B.Cu") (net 10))
 (segment (start 66.88 80) (end 67.46 80) (width 0.25) (layer "B.Cu") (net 10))
 (segment (start 64.88 80) (end 64.92 80) (width 0.25) (layer "B.Cu") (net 2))
 (segment (start 59.5 74.62) (end 64.88 80) (width 0.25) (layer "B.Cu") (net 2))
 (segment (start 80.054 93.934) (end 77.432715 93.934) (width 0.1) (layer "F.Cu") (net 14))
 (segment (start 82.595 96.475) (end 80.054 93.934) (width 0.1) (layer "F.Cu") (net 14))
 (segment (start 76.615 86.085) (end 77.62 85.08) (width 0.1) (layer "F.Cu") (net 14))
 (segment (start 76.615 93.116285) (end 76.615 86.085) (width 0.1) (layer "F.Cu") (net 14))
 (segment (start 77.432715 93.934) (end 76.615 93.116285) (width 0.1) (layer "F.Cu") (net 14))
 (segment (start 83.865 90.550001) (end 83.865 91.525) (width 0.1) (layer "F.Cu") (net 13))
 (segment (start 77.62 90.16) (end 83.474999 90.16) (width 0.1) (layer "F.Cu") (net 13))
 (segment (start 83.474999 90.16) (end 83.865 90.550001) (width 0.1) (layer "F.Cu") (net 13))
 (segment (start 86.405 90.258683) (end 86.405 91.525) (width 0.1) (layer "F.Cu") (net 11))
 (segment (start 77.62 82.54) (end 78.686317 82.54) (width 0.1) (layer "F.Cu") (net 11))
 (segment (start 78.686317 82.54) (end 86.405 90.258683) (width 0.1) (layer "F.Cu") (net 11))
 (segment (start 78.036285 94.235) (end 77.308037 94.235) (width 0.1) (layer "F.Cu") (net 15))
 (segment (start 81.502285 97.701) (end 78.036285 94.235) (width 0.1) (layer "F.Cu") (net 15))
 (segment (start 77.308037 94.235) (end 76.314 93.240963) (width 0.1) (layer "F.Cu") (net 15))
 (segment (start 76.314 81.306) (end 77.62 80) (width 0.1) (layer "F.Cu") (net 15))
 (segment (start 83.865 96.475) (end 83.865 96.751256) (width 0.1) (layer "F.Cu") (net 15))
 (segment (start 82.915256 97.701) (end 81.502285 97.701) (width 0.1) (layer "F.Cu") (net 15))
 (segment (start 83.865 96.751256) (end 82.915256 97.701) (width 0.1) (layer "F.Cu") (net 15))
 (segment (start 76.314 93.240963) (end 76.314 81.306) (width 0.1) (layer "F.Cu") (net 15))
 (segment (start 81.506256 87.62) (end 85.135 91.248744) (width 0.1) (layer "F.Cu") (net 12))
 (segment (start 85.135 91.248744) (end 85.135 91.525) (width 0.1) (layer "F.Cu") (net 12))
 (segment (start 77.62 87.62) (end 81.506256 87.62) (width 0.1) (layer "F.Cu") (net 12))
 (segment (start 85.27 96.95) (end 85.27 95.975001) (width 0.1) (layer "F.Cu") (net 16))
 (segment (start 82.5 95.5) (end 79.7 92.7) (width 0.1) (layer "F.Cu") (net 16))
 (segment (start 79.7 92.7) (end 77.62 92.7) (width 0.1) (layer "F.Cu") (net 16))
 (segment (start 77.62 92.7) (end 77.92 93) (width 0.1) (layer "F.Cu") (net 16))
 (segment (start 84.794999 95.5) (end 82.5 95.5) (width 0.1) (layer "F.Cu") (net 16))
 (segment (start 85.27 95.975001) (end 84.794999 95.5) (width 0.1) (layer "F.Cu") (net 16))
 (segment (start 68.5 67.19) (end 71.5 64.19) (width 0.2) (layer "F.Cu") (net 4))
 (segment (start 71.5 64.19) (end 71.5 53.1) (width 0.2) (layer "F.Cu") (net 4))
 (segment (start 78.7 82.092649) (end 78.7 99.24) (width 0.25) (layer "B.Cu") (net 3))
 (segment (start 68.54 80.54) (end 69.5 81.5) (width 0.25) (layer "B.Cu") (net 3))
 (segment (start 69.5 81.5) (end 76.5 81.5) (width 0.25) (layer "B.Cu") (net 3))
 (segment (start 68.54 74.85) (end 68.54 80.54) (width 0.25) (layer "B.Cu") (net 3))
 (segment (start 68.5 74.81) (end 68.54 74.85) (width 0.25) (layer "B.Cu") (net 3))
 (segment (start 76.54 81.46) (end 78.067351 81.46) (width 0.25) (layer "B.Cu") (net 3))
 (segment (start 76.5 81.5) (end 76.54 81.46) (width 0.25) (layer "B.Cu") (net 3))
 (segment (start 78.7 99.24) (end 77.62 100.32) (width 0.25) (layer "B.Cu") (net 3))
 (segment (start 78.067351 81.46) (end 78.7 82.092649) (width 0.25) (layer "B.Cu") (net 3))
 (segment (start 79.5 102.925678) (end 78.748678 103.677) (width 0.1) (layer "B.Cu") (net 8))
 (segment (start 80.628 87.5) (end 80.628 101.797678) (width 0.1) (layer "B.Cu") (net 8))
 (segment (start 81.323 86.677) (end 80.628 87.372) (width 0.1) (layer "B.Cu") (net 8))
 (segment (start 90.577 86.677) (end 81.5 86.677) (width 0.1) (layer "B.Cu") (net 8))
 (segment (start 77.581768 103.677) (end 75.199 101.294232) (width 0.1) (layer "B.Cu") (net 8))
 (segment (start 75.199 83.199) (end 75.102 83.102) (width 0.1) (layer "B.Cu") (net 8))
 (segment (start 63.5 89.04) (end 62.38 90.16) (width 0.1) (layer "B.Cu") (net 8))
 (segment (start 79.5 102.925678) (end 79.476678 102.949) (width 0.1) (layer "B.Cu") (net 8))
 (segment (start 63.5 83.5) (end 63.5 89.04) (width 0.1) (layer "B.Cu") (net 8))
 (segment (start 81.5 86.677) (end 81.323 86.677) (width 0.1) (layer "B.Cu") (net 8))
 (segment (start 78.748678 103.677) (end 77.581768 103.677) (width 0.1) (layer "B.Cu") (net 8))
 (segment (start 75.102 83.102) (end 63.898 83.102) (width 0.1) (layer "B.Cu") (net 8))
 (segment (start 75.199 101.294232) (end 75.199 83.199) (width 0.1) (layer "B.Cu") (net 8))
 (segment (start 80.628 87.372) (end 80.628 87.5) (width 0.1) (layer "B.Cu") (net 8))
 (segment (start 92.5 88.6) (end 90.577 86.677) (width 0.1) (layer "B.Cu") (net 8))
 (segment (start 63.898 83.102) (end 63.5 83.5) (width 0.1) (layer "B.Cu") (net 8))
 (segment (start 80.628 101.797678) (end 79.5 102.925678) (width 0.1) (layer "B.Cu") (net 8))
 (segment (start 77.706446 103.376) (end 75.5 101.169554) (width 0.1) (layer "B.Cu") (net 7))
 (segment (start 75.301 82.801) (end 66.801 82.801) (width 0.1) (layer "B.Cu") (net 7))
 (segment (start 81 86.376) (end 80.327 87.049) (width 0.1) (layer "B.Cu") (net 7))
 (segment (start 78.624 103.376) (end 77.706446 103.376) (width 0.1) (layer "B.Cu") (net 7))
 (segment (start 80.327 101.673) (end 78.624 103.376) (width 0.1) (layer "B.Cu") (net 7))
 (segment (start 59.075744 84.315744) (end 62.38 87.62) (width 0.1) (layer "B.Cu") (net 7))
 (segment (start 80.327 87.049) (end 80.327 101.673) (width 0.1) (layer "B.Cu") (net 7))
 (segment (start 66.801 82.801) (end 65.456 81.456) (width 0.1) (layer "B.Cu") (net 7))
 (segment (start 59.075744 81.456) (end 59.075744 84.315744) (width 0.1) (layer "B.Cu") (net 7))
 (segment (start 75.5 101.169554) (end 75.5 83) (width 0.1) (layer "B.Cu") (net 7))
 (segment (start 95.04 88.6) (end 92.816 86.376) (width 0.1) (layer "B.Cu") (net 7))
 (segment (start 92.816 86.376) (end 81 86.376) (width 0.1) (layer "B.Cu") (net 7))
 (segment (start 75.5 83) (end 75.301 82.801) (width 0.1) (layer "B.Cu") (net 7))
 (segment (start 65.456 81.456) (end 59.075744 81.456) (width 0.1) (layer "B.Cu") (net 7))
 (segment (start 58.27676 93.851) (end 55.12324 93.851) (width 0.1) (layer "B.Cu") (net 18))
 (segment (start 54.449 86.351) (end 55.6 85.2) (width 0.1) (layer "B.Cu") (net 18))
 (segment (start 55.12324 93.851) (end 54.449 93.17676) (width 0.1) (layer "B.Cu") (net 18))
 (segment (start 62.38 97.78) (end 62.20576 97.78) (width 0.1) (layer "B.Cu") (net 18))
 (segment (start 54.449 93.17676) (end 54.449 86.351) (width 0.1) (layer "B.Cu") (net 18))
 (segment (start 55.6 85.2) (end 56.7 85.2) (width 0.1) (layer "B.Cu") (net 18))
 (segment (start 62.20576 97.78) (end 58.27676 93.851) (width 0.1) (layer "B.Cu") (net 18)))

